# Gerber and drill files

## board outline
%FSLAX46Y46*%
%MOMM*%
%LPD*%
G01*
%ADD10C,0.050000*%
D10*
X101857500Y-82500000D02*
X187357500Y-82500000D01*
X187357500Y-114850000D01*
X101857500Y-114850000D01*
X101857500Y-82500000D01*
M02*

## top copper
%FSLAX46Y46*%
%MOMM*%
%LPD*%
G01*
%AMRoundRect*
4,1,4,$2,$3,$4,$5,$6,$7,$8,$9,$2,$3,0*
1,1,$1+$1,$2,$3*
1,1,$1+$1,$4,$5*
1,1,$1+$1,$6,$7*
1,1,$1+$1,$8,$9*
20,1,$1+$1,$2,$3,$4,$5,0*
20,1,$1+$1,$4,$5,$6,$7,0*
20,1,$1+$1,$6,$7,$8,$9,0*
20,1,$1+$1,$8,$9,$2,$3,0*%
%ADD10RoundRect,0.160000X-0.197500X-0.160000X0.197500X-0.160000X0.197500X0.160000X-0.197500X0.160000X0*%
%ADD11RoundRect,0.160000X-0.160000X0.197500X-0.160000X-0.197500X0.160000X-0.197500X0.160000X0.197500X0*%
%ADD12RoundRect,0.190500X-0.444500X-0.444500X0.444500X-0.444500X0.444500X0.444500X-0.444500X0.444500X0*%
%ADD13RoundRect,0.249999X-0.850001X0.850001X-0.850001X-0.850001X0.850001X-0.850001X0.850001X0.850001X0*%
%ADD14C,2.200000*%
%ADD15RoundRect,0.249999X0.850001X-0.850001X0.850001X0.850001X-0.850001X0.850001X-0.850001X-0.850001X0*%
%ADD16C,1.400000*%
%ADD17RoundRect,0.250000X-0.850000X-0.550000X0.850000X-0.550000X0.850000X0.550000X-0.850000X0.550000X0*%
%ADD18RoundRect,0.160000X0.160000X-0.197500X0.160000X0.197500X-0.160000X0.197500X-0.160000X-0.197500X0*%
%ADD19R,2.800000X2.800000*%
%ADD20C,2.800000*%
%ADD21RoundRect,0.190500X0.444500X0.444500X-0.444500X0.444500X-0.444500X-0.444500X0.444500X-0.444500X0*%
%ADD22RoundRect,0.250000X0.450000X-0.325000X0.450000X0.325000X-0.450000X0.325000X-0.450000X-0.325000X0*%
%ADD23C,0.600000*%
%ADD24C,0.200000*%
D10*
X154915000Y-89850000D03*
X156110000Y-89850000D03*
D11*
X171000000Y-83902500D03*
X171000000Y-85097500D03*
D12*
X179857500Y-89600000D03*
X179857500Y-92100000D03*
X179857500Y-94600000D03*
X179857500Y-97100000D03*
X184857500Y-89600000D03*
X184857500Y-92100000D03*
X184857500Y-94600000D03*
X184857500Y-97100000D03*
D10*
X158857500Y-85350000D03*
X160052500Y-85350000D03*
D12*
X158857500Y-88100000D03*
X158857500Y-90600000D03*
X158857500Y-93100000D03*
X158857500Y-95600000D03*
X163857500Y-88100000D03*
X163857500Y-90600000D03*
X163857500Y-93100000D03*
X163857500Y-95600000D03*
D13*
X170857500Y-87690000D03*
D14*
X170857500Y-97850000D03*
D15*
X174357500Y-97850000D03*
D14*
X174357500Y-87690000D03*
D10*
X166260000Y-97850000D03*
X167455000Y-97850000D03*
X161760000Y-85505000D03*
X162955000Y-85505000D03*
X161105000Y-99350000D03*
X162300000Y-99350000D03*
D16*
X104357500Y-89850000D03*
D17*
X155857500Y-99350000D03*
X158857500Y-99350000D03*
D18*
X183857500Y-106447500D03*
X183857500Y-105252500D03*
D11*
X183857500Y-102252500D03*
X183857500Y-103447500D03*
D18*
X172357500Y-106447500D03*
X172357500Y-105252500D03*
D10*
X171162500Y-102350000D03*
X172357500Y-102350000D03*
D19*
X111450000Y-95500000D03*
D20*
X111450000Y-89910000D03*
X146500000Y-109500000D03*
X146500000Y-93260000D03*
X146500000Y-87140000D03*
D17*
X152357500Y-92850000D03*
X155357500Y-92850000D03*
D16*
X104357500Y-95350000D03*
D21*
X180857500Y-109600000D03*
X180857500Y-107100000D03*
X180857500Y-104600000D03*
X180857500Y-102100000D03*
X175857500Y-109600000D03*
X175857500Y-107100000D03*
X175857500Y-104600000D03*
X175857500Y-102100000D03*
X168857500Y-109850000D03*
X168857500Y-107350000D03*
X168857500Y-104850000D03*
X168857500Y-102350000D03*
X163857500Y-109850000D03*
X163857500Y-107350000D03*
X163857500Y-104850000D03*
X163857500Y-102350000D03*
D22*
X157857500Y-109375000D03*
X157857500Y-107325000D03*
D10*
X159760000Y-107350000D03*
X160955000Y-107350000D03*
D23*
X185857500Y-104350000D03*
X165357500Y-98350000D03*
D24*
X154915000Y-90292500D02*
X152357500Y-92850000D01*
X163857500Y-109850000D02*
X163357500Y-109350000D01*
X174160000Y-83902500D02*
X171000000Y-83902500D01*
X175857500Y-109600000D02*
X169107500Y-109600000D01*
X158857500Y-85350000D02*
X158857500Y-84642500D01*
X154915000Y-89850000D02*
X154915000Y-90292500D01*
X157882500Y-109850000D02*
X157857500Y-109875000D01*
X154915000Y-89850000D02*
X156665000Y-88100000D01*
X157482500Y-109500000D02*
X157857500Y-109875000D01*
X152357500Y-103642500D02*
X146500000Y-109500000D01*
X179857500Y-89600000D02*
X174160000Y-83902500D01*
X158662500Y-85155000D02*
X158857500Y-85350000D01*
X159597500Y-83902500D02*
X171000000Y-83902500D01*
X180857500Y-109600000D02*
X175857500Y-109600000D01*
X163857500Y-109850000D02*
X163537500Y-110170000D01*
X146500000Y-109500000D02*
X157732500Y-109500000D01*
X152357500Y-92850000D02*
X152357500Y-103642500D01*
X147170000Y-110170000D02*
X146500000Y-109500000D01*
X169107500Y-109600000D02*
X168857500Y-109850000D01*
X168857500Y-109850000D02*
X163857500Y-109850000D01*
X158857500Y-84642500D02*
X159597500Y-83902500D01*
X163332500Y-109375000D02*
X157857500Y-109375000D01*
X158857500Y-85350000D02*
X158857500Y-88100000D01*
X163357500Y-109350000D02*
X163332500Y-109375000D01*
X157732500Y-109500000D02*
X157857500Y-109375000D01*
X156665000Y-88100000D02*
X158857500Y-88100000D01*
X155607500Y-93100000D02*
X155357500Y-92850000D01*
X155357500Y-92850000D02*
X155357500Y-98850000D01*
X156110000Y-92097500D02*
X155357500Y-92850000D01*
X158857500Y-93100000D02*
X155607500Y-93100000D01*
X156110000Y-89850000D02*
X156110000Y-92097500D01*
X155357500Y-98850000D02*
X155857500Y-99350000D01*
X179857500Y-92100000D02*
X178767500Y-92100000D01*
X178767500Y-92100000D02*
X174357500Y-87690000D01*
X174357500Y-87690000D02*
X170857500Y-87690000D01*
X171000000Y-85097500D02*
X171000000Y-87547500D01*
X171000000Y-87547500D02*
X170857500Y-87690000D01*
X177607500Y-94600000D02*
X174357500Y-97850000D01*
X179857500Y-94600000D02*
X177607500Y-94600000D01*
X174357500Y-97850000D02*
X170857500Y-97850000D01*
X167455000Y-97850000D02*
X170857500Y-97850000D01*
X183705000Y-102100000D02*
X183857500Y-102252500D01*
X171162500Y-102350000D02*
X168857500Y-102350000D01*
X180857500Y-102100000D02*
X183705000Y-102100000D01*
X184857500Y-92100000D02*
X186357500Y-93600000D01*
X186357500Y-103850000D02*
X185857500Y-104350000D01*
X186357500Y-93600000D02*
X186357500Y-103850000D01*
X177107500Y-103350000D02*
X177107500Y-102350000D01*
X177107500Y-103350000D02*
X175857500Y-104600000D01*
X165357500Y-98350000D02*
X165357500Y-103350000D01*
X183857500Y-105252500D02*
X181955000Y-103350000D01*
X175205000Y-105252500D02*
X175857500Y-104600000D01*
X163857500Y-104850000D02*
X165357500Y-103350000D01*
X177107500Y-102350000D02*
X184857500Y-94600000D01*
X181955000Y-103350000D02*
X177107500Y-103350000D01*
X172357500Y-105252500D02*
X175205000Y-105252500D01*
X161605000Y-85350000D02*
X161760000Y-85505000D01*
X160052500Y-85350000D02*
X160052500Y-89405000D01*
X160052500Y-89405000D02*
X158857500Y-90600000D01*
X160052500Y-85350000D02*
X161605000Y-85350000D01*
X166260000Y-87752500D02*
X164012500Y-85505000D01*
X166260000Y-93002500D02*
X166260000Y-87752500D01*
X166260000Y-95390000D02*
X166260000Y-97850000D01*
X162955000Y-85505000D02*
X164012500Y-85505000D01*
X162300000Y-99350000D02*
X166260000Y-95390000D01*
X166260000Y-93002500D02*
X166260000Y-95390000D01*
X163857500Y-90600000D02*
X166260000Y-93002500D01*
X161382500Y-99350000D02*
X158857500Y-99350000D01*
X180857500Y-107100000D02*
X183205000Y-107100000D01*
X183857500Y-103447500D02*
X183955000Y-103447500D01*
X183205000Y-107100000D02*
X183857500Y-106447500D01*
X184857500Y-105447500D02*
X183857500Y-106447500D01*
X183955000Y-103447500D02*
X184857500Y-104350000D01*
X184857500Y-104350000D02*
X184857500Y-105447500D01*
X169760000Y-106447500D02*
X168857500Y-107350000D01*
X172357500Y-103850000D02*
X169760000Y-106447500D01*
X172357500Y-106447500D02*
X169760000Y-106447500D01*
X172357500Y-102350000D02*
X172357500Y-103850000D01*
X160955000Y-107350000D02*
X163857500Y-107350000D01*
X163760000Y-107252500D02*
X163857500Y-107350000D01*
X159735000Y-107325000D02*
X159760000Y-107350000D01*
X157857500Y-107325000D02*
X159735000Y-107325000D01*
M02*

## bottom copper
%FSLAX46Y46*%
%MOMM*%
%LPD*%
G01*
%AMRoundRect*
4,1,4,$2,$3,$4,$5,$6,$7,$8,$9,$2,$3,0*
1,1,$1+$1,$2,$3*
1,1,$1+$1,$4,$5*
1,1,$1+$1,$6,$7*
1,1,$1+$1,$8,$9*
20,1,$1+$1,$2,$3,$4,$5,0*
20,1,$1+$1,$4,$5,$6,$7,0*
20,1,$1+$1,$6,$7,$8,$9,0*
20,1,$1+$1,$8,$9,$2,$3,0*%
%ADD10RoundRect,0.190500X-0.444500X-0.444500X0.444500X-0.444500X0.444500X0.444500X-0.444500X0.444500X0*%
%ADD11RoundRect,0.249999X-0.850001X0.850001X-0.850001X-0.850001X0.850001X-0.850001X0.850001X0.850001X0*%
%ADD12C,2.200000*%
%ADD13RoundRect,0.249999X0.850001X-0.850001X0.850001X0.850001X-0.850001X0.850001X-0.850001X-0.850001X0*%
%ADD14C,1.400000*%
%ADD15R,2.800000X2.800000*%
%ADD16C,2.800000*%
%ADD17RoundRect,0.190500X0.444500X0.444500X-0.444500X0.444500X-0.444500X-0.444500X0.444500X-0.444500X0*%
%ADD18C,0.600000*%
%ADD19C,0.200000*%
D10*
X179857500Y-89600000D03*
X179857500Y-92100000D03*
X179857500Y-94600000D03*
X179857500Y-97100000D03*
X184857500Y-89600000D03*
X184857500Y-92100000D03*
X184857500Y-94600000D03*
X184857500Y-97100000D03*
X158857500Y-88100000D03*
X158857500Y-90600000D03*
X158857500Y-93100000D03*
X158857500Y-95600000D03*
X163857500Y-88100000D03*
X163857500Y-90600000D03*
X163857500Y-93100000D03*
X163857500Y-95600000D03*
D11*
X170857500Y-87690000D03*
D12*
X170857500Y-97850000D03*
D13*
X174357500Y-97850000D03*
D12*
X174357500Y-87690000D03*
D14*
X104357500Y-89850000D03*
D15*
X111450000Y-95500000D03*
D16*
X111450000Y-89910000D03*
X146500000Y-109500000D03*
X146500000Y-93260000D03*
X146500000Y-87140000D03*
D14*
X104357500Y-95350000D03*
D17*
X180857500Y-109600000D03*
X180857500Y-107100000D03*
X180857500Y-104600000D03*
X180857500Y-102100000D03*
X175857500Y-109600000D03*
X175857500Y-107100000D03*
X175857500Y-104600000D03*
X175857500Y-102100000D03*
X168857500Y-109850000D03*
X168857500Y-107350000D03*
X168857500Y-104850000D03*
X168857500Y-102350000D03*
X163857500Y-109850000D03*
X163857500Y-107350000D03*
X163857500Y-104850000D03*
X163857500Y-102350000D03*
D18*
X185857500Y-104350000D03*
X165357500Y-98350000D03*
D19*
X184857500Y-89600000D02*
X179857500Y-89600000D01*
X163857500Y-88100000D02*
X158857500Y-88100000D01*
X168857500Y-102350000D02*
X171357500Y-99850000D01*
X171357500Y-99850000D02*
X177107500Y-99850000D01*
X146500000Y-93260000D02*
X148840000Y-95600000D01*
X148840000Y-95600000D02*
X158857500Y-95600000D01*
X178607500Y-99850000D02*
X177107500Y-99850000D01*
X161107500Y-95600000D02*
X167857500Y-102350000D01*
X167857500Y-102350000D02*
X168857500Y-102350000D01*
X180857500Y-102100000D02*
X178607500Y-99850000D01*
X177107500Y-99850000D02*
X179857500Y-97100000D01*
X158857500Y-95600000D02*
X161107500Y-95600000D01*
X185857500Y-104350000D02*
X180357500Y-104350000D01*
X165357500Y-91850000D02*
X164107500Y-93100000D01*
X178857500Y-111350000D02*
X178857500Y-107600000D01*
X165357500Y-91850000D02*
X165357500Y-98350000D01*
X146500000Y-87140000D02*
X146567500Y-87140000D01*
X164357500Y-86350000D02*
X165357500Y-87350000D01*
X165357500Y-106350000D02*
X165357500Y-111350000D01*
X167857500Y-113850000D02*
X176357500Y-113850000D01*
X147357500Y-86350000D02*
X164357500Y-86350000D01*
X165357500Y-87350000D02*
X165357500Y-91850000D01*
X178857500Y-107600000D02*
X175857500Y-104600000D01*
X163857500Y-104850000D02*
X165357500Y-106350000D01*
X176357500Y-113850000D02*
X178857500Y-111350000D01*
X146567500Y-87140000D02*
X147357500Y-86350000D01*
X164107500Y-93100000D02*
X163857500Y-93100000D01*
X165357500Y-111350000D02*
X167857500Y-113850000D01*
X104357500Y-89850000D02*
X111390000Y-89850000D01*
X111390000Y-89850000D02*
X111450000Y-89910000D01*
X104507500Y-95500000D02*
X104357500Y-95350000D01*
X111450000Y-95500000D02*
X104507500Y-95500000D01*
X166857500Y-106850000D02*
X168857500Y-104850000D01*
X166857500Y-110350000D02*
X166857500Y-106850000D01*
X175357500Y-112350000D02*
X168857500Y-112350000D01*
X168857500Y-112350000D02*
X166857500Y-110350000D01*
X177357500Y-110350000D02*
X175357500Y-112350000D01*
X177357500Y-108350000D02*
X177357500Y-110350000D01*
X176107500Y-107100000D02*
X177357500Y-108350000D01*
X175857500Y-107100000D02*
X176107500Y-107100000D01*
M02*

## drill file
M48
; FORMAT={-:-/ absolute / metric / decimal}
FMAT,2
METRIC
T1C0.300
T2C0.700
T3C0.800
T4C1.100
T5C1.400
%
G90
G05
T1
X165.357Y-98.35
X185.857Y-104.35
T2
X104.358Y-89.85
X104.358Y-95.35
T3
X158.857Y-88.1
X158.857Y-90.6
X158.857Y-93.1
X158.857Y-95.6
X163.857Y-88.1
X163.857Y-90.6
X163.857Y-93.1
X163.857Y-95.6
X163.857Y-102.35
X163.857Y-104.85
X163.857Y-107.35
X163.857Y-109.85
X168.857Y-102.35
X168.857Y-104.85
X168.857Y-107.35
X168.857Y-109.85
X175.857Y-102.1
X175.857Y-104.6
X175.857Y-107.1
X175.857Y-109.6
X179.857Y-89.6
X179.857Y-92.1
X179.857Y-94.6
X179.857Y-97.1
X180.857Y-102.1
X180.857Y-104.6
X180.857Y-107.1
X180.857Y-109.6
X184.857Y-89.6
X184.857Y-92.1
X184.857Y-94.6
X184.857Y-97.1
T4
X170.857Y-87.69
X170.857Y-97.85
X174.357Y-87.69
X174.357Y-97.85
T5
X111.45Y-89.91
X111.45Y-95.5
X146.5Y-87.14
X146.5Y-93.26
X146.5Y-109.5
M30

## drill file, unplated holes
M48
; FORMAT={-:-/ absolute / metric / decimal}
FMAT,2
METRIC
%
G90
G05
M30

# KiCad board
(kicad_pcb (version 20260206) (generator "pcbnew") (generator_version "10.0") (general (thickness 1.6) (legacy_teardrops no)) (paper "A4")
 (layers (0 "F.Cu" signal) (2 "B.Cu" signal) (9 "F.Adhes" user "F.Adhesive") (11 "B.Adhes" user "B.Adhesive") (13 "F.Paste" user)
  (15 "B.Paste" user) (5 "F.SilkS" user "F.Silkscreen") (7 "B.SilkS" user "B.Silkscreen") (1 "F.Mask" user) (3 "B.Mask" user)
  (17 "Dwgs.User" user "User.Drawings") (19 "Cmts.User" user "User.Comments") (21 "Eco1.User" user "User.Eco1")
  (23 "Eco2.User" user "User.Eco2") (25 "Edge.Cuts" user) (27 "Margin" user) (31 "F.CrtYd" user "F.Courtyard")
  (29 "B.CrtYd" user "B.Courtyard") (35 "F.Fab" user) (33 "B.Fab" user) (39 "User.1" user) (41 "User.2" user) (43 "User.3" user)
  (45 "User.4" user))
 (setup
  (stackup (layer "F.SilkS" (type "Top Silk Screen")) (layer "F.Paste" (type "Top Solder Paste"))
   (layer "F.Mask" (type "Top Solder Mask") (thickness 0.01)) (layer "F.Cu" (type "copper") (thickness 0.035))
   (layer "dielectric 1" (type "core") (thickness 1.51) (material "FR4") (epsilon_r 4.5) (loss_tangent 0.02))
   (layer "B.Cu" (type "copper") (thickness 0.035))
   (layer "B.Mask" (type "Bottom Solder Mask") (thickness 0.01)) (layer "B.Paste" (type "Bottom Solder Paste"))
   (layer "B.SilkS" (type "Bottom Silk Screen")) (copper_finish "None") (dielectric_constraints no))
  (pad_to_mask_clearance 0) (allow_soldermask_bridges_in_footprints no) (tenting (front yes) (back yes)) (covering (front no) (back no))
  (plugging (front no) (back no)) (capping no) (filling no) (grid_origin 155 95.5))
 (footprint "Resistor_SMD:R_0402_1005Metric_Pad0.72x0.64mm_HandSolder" (layer "F.Cu") (at 155.5125 89.85)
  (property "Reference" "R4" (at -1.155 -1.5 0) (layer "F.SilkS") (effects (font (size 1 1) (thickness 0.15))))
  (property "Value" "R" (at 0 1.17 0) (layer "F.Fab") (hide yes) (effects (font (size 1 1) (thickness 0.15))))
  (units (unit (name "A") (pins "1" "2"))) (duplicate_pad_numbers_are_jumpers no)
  (pad "1" smd roundrect (at -0.5975 0) (size 0.715 0.64) (layers "F.Cu" "F.Mask" "F.Paste") (roundrect_rratio 0.25) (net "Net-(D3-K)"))
  (pad "2" smd roundrect (at 0.5975 0) (size 0.715 0.64) (layers "F.Cu" "F.Mask" "F.Paste") (roundrect_rratio 0.25) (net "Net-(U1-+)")))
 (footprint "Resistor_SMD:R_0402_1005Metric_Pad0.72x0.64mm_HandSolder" (layer "F.Cu") (at 171 84.5 -90)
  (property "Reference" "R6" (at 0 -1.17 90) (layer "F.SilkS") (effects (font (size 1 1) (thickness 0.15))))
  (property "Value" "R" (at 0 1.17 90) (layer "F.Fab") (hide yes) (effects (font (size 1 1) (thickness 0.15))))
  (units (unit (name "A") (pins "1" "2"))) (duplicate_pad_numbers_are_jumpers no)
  (pad "1" smd roundrect (at -0.5975 0 270) (size 0.715 0.64) (layers "F.Cu" "F.Mask" "F.Paste") (roundrect_rratio 0.25) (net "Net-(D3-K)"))
  (pad "2" smd roundrect (at 0.5975 0 270) (size 0.715 0.64) (layers "F.Cu" "F.Mask" "F.Paste") (roundrect_rratio 0.25) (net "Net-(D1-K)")))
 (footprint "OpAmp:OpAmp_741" (layer "F.Cu") (at 182.3575 96.1)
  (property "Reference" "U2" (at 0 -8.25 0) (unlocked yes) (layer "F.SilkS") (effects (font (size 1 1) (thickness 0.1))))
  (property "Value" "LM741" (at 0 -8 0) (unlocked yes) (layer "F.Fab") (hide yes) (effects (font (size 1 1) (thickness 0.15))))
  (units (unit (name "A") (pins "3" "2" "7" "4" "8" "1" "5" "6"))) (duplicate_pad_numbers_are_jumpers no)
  (pad "1" thru_hole roundrect (at -2.5 -6.5) (size 1.27 1.27) (drill 0.8) (layers "*.Cu" "*.Mask") (remove_unused_layers no)
   (roundrect_rratio 0.15) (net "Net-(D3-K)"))
  (pad "2" thru_hole roundrect (at -2.5 -4) (size 1.27 1.27) (drill 0.8) (layers "*.Cu" "*.Mask") (remove_unused_layers no)
   (roundrect_rratio 0.15) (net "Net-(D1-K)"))
  (pad "3" thru_hole roundrect (at -2.5 -1.5) (size 1.27 1.27) (drill 0.8) (layers "*.Cu" "*.Mask") (remove_unused_layers no)
   (roundrect_rratio 0.15) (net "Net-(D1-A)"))
  (pad "4" thru_hole roundrect (at -2.5 1) (size 1.27 1.27) (drill 0.8) (layers "*.Cu" "*.Mask") (remove_unused_layers no)
   (roundrect_rratio 0.15) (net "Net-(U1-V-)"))
  (pad "5" thru_hole roundrect (at 2.5 -6.5) (size 1.27 1.27) (drill 0.8) (layers "*.Cu" "*.Mask") (remove_unused_layers no)
   (roundrect_rratio 0.15) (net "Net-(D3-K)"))
  (pad "6" thru_hole roundrect (at 2.5 -4) (size 1.27 1.27) (drill 0.8) (layers "*.Cu" "*.Mask") (remove_unused_layers no)
   (roundrect_rratio 0.15) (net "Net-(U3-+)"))
  (pad "7" thru_hole roundrect (at 2.5 -1.5) (size 1.27 1.27) (drill 0.8) (layers "*.Cu" "*.Mask") (remove_unused_layers no)
   (roundrect_rratio 0.15) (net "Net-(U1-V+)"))
  (pad "8" thru_hole roundrect (at 2.5 1) (size 1.27 1.27) (drill 0.8) (layers "*.Cu" "*.Mask") (remove_unused_layers no)
   (roundrect_rratio 0.15) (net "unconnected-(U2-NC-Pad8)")))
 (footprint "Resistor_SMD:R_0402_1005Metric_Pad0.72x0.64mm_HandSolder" (layer "F.Cu") (at 159.455 85.35)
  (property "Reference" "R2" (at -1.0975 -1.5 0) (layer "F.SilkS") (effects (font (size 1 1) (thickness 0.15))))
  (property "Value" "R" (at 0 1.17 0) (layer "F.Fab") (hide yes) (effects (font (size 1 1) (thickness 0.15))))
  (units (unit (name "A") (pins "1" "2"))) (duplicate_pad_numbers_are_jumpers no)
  (pad "1" smd roundrect (at -0.5975 0) (size 0.715 0.64) (layers "F.Cu" "F.Mask" "F.Paste") (roundrect_rratio 0.25) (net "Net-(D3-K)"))
  (pad "2" smd roundrect (at 0.5975 0) (size 0.715 0.64) (layers "F.Cu" "F.Mask" "F.Paste") (roundrect_rratio 0.25) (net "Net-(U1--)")))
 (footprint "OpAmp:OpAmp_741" (layer "F.Cu") (at 161.3575 94.6)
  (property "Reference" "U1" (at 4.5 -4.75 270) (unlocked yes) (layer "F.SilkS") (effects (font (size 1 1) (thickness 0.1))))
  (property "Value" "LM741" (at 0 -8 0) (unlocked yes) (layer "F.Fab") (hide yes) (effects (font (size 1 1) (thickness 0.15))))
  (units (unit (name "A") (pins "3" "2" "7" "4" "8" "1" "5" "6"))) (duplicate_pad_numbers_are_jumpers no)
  (pad "1" thru_hole roundrect (at -2.5 -6.5) (size 1.27 1.27) (drill 0.8) (layers "*.Cu" "*.Mask") (remove_unused_layers no)
   (roundrect_rratio 0.15) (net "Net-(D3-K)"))
  (pad "2" thru_hole roundrect (at -2.5 -4) (size 1.27 1.27) (drill 0.8) (layers "*.Cu" "*.Mask") (remove_unused_layers no)
   (roundrect_rratio 0.15) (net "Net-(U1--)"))
  (pad "3" thru_hole roundrect (at -2.5 -1.5) (size 1.27 1.27) (drill 0.8) (layers "*.Cu" "*.Mask") (remove_unused_layers no)
   (roundrect_rratio 0.15) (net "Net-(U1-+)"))
  (pad "4" thru_hole roundrect (at -2.5 1) (size 1.27 1.27) (drill 0.8) (layers "*.Cu" "*.Mask") (remove_unused_layers no)
   (roundrect_rratio 0.15) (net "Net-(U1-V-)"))
  (pad "5" thru_hole roundrect (at 2.5 -6.5) (size 1.27 1.27) (drill 0.8) (layers "*.Cu" "*.Mask") (remove_unused_layers no)
   (roundrect_rratio 0.15) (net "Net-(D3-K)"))
  (pad "6" thru_hole roundrect (at 2.5 -4) (size 1.27 1.27) (drill 0.8) (layers "*.Cu" "*.Mask") (remove_unused_layers no)
   (roundrect_rratio 0.15) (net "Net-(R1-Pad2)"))
  (pad "7" thru_hole roundrect (at 2.5 -1.5) (size 1.27 1.27) (drill 0.8) (layers "*.Cu" "*.Mask") (remove_unused_layers no)
   (roundrect_rratio 0.15) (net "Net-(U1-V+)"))
  (pad "8" thru_hole roundrect (at 2.5 1) (size 1.27 1.27) (drill 0.8) (layers "*.Cu" "*.Mask") (remove_unused_layers no)
   (roundrect_rratio 0.15) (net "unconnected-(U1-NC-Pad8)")))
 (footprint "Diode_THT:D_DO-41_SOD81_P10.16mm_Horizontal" (layer "F.Cu") (at 170.8575 87.69 -90)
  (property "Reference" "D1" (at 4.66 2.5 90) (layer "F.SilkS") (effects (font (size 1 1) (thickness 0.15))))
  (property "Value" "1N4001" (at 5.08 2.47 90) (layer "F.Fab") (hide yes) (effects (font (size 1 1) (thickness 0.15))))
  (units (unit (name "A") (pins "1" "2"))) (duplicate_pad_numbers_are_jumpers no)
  (pad "1" thru_hole roundrect (at 0 0 270) (size 2.2 2.2) (drill 1.1) (layers "*.Cu" "*.Mask") (remove_unused_layers no)
   (roundrect_rratio 0.113636) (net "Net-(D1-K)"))
  (pad "2" thru_hole circle (at 10.16 0 270) (size 2.2 2.2) (drill 1.1) (layers "*.Cu" "*.Mask") (remove_unused_layers no)
   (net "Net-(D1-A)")))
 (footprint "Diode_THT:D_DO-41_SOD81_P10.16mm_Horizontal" (layer "F.Cu") (at 174.3575 97.85 90)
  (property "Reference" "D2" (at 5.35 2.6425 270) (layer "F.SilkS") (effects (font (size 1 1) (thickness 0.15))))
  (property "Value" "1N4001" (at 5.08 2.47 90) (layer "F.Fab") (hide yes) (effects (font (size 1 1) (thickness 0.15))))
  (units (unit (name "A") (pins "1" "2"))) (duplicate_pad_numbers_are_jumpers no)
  (pad "1" thru_hole roundrect (at 0 0 90) (size 2.2 2.2) (drill 1.1) (layers "*.Cu" "*.Mask") (remove_unused_layers no)
   (roundrect_rratio 0.113636) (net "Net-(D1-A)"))
  (pad "2" thru_hole circle (at 10.16 0 90) (size 2.2 2.2) (drill 1.1) (layers "*.Cu" "*.Mask") (remove_unused_layers no) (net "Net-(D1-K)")))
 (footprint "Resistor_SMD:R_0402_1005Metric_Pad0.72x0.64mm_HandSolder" (layer "F.Cu") (at 166.8575 97.85)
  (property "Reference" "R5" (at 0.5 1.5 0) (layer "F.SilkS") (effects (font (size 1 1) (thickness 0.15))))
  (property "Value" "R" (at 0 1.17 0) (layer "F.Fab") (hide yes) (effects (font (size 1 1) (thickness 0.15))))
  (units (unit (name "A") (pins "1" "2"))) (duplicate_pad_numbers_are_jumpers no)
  (pad "1" smd roundrect (at -0.5975 0) (size 0.715 0.64) (layers "F.Cu" "F.Mask" "F.Paste") (roundrect_rratio 0.25) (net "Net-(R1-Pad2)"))
  (pad "2" smd roundrect (at 0.5975 0) (size 0.715 0.64) (layers "F.Cu" "F.Mask" "F.Paste") (roundrect_rratio 0.25) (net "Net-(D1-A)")))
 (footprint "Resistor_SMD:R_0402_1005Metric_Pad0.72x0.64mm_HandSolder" (layer "F.Cu") (at 162.3575 85.505)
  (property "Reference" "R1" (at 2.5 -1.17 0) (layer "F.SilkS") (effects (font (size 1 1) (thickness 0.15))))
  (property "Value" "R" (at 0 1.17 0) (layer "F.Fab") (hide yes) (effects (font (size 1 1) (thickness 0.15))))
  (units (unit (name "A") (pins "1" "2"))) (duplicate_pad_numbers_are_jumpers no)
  (pad "1" smd roundrect (at -0.5975 0) (size 0.715 0.64) (layers "F.Cu" "F.Mask" "F.Paste") (roundrect_rratio 0.25) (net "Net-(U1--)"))
  (pad "2" smd roundrect (at 0.5975 0) (size 0.715 0.64) (layers "F.Cu" "F.Mask" "F.Paste") (roundrect_rratio 0.25) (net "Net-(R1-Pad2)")))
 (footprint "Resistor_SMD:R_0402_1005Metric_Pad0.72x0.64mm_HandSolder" (layer "F.Cu") (at 161.7025 99.35)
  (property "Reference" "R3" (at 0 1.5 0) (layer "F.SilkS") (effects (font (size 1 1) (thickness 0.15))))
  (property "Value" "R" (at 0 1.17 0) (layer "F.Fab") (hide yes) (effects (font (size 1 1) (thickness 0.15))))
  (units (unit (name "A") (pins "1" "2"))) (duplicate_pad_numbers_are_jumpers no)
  (pad "1" smd roundrect (at -0.5975 0) (size 0.715 0.64) (layers "F.Cu" "F.Mask" "F.Paste") (roundrect_rratio 0.25) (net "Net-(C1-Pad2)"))
  (pad "2" smd roundrect (at 0.5975 0) (size 0.715 0.64) (layers "F.Cu" "F.Mask" "F.Paste") (roundrect_rratio 0.25) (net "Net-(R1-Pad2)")))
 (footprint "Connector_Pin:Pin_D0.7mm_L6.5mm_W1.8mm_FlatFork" (layer "F.Cu") (at 104.3575 89.85)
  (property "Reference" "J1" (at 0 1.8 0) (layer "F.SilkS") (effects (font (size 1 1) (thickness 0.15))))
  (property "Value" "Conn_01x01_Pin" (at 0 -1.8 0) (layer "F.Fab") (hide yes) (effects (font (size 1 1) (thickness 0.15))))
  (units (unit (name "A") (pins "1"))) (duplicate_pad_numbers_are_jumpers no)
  (pad "1" thru_hole circle (at 0 0) (size 1.4 1.4) (drill 0.7) (layers "*.Cu" "*.Mask") (remove_unused_layers no) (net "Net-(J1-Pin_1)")))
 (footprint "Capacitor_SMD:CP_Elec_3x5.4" (layer "F.Cu") (at 157.3575 99.35)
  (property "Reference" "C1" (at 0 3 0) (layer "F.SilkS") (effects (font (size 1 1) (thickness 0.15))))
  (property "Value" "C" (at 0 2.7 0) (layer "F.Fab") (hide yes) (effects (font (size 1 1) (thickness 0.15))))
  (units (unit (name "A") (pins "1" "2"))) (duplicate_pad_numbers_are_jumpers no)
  (pad "1" smd roundrect (at -1.5 0) (size 2.2 1.6) (layers "F.Cu" "F.Mask" "F.Paste") (roundrect_rratio 0.15625) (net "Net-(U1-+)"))
  (pad "2" smd roundrect (at 1.5 0) (size 2.2 1.6) (layers "F.Cu" "F.Mask" "F.Paste") (roundrect_rratio 0.15625) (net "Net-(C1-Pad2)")))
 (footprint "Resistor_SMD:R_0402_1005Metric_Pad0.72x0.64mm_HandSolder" (layer "F.Cu") (at 183.8575 105.85 90)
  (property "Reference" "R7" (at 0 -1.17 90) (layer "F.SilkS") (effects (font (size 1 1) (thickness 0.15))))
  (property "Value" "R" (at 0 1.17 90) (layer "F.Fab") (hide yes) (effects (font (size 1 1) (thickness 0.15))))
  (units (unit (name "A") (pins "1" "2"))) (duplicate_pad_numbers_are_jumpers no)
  (pad "1" smd roundrect (at -0.5975 0 90) (size 0.715 0.64) (layers "F.Cu" "F.Mask" "F.Paste") (roundrect_rratio 0.25) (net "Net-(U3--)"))
  (pad "2" smd roundrect (at 0.5975 0 90) (size 0.715 0.64) (layers "F.Cu" "F.Mask" "F.Paste") (roundrect_rratio 0.25) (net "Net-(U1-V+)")))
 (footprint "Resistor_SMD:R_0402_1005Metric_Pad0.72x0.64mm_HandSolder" (layer "F.Cu") (at 183.8575 102.85 -90)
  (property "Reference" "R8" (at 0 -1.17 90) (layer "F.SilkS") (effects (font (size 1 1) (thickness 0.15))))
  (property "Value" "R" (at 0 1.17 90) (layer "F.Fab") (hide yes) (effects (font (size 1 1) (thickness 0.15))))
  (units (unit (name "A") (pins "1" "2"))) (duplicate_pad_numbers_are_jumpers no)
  (pad "1" smd roundrect (at -0.5975 0 270) (size 0.715 0.64) (layers "F.Cu" "F.Mask" "F.Paste") (roundrect_rratio 0.25) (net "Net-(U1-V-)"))
  (pad "2" smd roundrect (at 0.5975 0 270) (size 0.715 0.64) (layers "F.Cu" "F.Mask" "F.Paste") (roundrect_rratio 0.25) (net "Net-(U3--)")))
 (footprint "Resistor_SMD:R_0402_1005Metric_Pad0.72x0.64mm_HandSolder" (layer "F.Cu") (at 172.3575 105.85 90)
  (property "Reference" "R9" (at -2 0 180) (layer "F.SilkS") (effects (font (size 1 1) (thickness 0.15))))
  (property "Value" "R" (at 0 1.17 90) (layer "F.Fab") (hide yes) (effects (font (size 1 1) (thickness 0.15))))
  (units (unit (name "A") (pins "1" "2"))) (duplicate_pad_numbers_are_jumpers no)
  (pad "1" smd roundrect (at -0.5975 0 90) (size 0.715 0.64) (layers "F.Cu" "F.Mask" "F.Paste") (roundrect_rratio 0.25) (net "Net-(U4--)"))
  (pad "2" smd roundrect (at 0.5975 0 90) (size 0.715 0.64) (layers "F.Cu" "F.Mask" "F.Paste") (roundrect_rratio 0.25) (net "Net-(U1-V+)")))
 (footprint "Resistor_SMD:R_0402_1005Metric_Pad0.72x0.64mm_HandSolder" (layer "F.Cu") (at 171.76 102.35)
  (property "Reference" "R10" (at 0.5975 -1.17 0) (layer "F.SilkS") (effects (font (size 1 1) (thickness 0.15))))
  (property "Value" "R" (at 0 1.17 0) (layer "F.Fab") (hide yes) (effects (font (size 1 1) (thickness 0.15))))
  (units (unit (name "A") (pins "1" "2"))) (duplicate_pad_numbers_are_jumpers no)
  (pad "1" smd roundrect (at -0.5975 0) (size 0.715 0.64) (layers "F.Cu" "F.Mask" "F.Paste") (roundrect_rratio 0.25) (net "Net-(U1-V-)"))
  (pad "2" smd roundrect (at 0.5975 0) (size 0.715 0.64) (layers "F.Cu" "F.Mask" "F.Paste") (roundrect_rratio 0.25) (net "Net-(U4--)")))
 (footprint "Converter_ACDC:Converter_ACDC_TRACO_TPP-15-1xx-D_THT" (layer "F.Cu") (at 111.45 95.5)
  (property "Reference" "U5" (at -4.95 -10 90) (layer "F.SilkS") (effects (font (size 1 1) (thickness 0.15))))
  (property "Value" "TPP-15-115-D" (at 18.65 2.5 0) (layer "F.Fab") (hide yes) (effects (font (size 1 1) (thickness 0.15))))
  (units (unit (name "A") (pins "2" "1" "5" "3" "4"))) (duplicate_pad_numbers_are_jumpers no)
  (pad "1" thru_hole rect (at 0 0) (size 2.8 2.8) (drill 1.4) (layers "*.Cu" "*.Mask") (remove_unused_layers no) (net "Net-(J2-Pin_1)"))
  (pad "2" thru_hole circle (at 0 -5.59) (size 2.8 2.8) (drill 1.4) (layers "*.Cu" "*.Mask") (remove_unused_layers no)
   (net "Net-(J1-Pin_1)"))
  (pad "3" thru_hole circle (at 35.05 14) (size 2.8 2.8) (drill 1.4) (layers "*.Cu" "*.Mask") (remove_unused_layers no) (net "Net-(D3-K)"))
  (pad "4" thru_hole circle (at 35.05 -2.24) (size 2.8 2.8) (drill 1.4) (layers "*.Cu" "*.Mask") (remove_unused_layers no)
   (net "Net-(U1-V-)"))
  (pad "5" thru_hole circle (at 35.05 -8.36) (size 2.8 2.8) (drill 1.4) (layers "*.Cu" "*.Mask") (remove_unused_layers no)
   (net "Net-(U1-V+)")))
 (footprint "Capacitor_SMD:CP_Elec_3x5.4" (layer "F.Cu") (at 153.8575 92.85)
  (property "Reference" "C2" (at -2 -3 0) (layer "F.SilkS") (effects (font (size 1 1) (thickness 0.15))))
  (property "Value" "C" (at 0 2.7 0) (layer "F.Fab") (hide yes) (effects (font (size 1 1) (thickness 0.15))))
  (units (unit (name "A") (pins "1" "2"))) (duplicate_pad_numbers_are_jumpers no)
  (pad "1" smd roundrect (at -1.5 0) (size 2.2 1.6) (layers "F.Cu" "F.Mask" "F.Paste") (roundrect_rratio 0.15625) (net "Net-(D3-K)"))
  (pad "2" smd roundrect (at 1.5 0) (size 2.2 1.6) (layers "F.Cu" "F.Mask" "F.Paste") (roundrect_rratio 0.15625) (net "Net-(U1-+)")))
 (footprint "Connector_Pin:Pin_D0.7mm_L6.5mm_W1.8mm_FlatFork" (layer "F.Cu") (at 104.3575 95.35)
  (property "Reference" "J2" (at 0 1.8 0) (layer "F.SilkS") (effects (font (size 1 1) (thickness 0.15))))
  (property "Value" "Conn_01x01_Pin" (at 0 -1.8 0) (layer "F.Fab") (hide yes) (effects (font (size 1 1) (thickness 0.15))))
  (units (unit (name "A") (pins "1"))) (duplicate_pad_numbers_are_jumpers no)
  (pad "1" thru_hole circle (at 0 0) (size 1.4 1.4) (drill 0.7) (layers "*.Cu" "*.Mask") (remove_unused_layers no) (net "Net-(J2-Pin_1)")))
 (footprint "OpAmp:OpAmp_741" (layer "F.Cu") (at 178.3575 103.1 180)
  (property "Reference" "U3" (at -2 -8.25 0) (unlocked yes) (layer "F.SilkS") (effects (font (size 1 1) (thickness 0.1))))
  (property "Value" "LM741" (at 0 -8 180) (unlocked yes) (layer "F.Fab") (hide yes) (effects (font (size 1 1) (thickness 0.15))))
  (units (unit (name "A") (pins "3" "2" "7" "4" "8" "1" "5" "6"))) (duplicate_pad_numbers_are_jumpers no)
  (pad "1" thru_hole roundrect (at -2.5 -6.5 180) (size 1.27 1.27) (drill 0.8) (layers "*.Cu" "*.Mask") (remove_unused_layers no)
   (roundrect_rratio 0.15) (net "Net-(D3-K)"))
  (pad "2" thru_hole roundrect (at -2.5 -4 180) (size 1.27 1.27) (drill 0.8) (layers "*.Cu" "*.Mask") (remove_unused_layers no)
   (roundrect_rratio 0.15) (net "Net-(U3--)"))
  (pad "3" thru_hole roundrect (at -2.5 -1.5 180) (size 1.27 1.27) (drill 0.8) (layers "*.Cu" "*.Mask") (remove_unused_layers no)
   (roundrect_rratio 0.15) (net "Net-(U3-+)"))
  (pad "4" thru_hole roundrect (at -2.5 1 180) (size 1.27 1.27) (drill 0.8) (layers "*.Cu" "*.Mask") (remove_unused_layers no)
   (roundrect_rratio 0.15) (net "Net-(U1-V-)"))
  (pad "5" thru_hole roundrect (at 2.5 -6.5 180) (size 1.27 1.27) (drill 0.8) (layers "*.Cu" "*.Mask") (remove_unused_layers no)
   (roundrect_rratio 0.15) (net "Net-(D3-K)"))
  (pad "6" thru_hole roundrect (at 2.5 -4 180) (size 1.27 1.27) (drill 0.8) (layers "*.Cu" "*.Mask") (remove_unused_layers no)
   (roundrect_rratio 0.15) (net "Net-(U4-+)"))
  (pad "7" thru_hole roundrect (at 2.5 -1.5 180) (size 1.27 1.27) (drill 0.8) (layers "*.Cu" "*.Mask") (remove_unused_layers no)
   (roundrect_rratio 0.15) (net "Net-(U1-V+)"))
  (pad "8" thru_hole roundrect (at 2.5 1 180) (size 1.27 1.27) (drill 0.8) (layers "*.Cu" "*.Mask") (remove_unused_layers no)
   (roundrect_rratio 0.15) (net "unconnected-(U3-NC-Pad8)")))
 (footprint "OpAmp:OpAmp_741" (layer "F.Cu") (at 166.3575 103.35 180)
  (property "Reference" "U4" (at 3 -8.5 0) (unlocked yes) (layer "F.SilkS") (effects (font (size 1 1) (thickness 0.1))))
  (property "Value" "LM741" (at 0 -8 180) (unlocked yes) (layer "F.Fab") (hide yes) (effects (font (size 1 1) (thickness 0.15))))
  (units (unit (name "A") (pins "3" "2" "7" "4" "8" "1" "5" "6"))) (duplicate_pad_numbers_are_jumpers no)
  (pad "1" thru_hole roundrect (at -2.5 -6.5 180) (size 1.27 1.27) (drill 0.8) (layers "*.Cu" "*.Mask") (remove_unused_layers no)
   (roundrect_rratio 0.15) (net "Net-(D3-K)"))
  (pad "2" thru_hole roundrect (at -2.5 -4 180) (size 1.27 1.27) (drill 0.8) (layers "*.Cu" "*.Mask") (remove_unused_layers no)
   (roundrect_rratio 0.15) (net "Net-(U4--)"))
  (pad "3" thru_hole roundrect (at -2.5 -1.5 180) (size 1.27 1.27) (drill 0.8) (layers "*.Cu" "*.Mask") (remove_unused_layers no)
   (roundrect_rratio 0.15) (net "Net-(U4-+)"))
  (pad "4" thru_hole roundrect (at -2.5 1 180) (size 1.27 1.27) (drill 0.8) (layers "*.Cu" "*.Mask") (remove_unused_layers no)
   (roundrect_rratio 0.15) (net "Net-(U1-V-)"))
  (pad "5" thru_hole roundrect (at 2.5 -6.5 180) (size 1.27 1.27) (drill 0.8) (layers "*.Cu" "*.Mask") (remove_unused_layers no)
   (roundrect_rratio 0.15) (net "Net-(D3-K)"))
  (pad "6" thru_hole roundrect (at 2.5 -4 180) (size 1.27 1.27) (drill 0.8) (layers "*.Cu" "*.Mask") (remove_unused_layers no)
   (roundrect_rratio 0.15) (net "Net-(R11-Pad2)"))
  (pad "7" thru_hole roundrect (at 2.5 -1.5 180) (size 1.27 1.27) (drill 0.8) (layers "*.Cu" "*.Mask") (remove_unused_layers no)
   (roundrect_rratio 0.15) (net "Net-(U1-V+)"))
  (pad "8" thru_hole roundrect (at 2.5 1 180) (size 1.27 1.27) (drill 0.8) (layers "*.Cu" "*.Mask") (remove_unused_layers no)
   (roundrect_rratio 0.15) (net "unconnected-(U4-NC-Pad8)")))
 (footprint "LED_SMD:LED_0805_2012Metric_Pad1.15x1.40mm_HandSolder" (layer "F.Cu") (at 157.8575 108.35 90)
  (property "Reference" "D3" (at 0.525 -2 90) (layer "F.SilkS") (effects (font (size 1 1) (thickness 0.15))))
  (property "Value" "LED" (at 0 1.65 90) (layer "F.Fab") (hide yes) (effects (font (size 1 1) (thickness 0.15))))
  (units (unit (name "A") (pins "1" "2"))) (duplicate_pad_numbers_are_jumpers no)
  (pad "1" smd roundrect (at -1.025 0 90) (size 1.15 1.4) (layers "F.Cu" "F.Mask" "F.Paste") (roundrect_rratio 0.217391) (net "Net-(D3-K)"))
  (pad "2" smd roundrect (at 1.025 0 90) (size 1.15 1.4) (layers "F.Cu" "F.Mask" "F.Paste") (roundrect_rratio 0.217391) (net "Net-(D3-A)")))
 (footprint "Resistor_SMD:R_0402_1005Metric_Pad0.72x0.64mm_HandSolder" (layer "F.Cu") (at 160.3575 107.35)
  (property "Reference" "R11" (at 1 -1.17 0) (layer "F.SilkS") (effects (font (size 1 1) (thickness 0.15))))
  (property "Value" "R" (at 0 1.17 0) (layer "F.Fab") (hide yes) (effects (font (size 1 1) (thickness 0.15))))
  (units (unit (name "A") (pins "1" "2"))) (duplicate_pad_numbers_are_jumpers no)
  (pad "1" smd roundrect (at -0.5975 0) (size 0.715 0.64) (layers "F.Cu" "F.Mask" "F.Paste") (roundrect_rratio 0.25) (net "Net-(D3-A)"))
  (pad "2" smd roundrect (at 0.5975 0) (size 0.715 0.64) (layers "F.Cu" "F.Mask" "F.Paste") (roundrect_rratio 0.25) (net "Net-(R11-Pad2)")))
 (gr_rect (start 101.8575 82.5) (end 187.3575 114.85) (stroke (width 0.05) (type default)) (fill no) (layer "Edge.Cuts"))
 (segment (start 154.915 90.2925) (end 152.3575 92.85) (width 0.2) (layer "F.Cu") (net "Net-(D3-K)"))
 (segment (start 163.8575 109.85) (end 163.3575 109.35) (width 0.2) (layer "F.Cu") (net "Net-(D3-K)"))
 (segment (start 174.16 83.9025) (end 171 83.9025) (width 0.2) (layer "F.Cu") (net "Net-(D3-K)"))
 (segment (start 175.8575 109.6) (end 169.1075 109.6) (width 0.2) (layer "F.Cu") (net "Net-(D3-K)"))
 (segment (start 158.8575 85.35) (end 158.8575 84.6425) (width 0.2) (layer "F.Cu") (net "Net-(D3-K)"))
 (segment (start 154.915 89.85) (end 154.915 90.2925) (width 0.2) (layer "F.Cu") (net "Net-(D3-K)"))
 (segment (start 157.8825 109.85) (end 157.8575 109.875) (width 0.2) (layer "F.Cu") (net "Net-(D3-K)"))
 (segment (start 154.915 89.85) (end 156.665 88.1) (width 0.2) (layer "F.Cu") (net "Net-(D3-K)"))
 (segment (start 157.4825 109.5) (end 157.8575 109.875) (width 0.2) (layer "F.Cu") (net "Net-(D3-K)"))
 (segment (start 152.3575 103.6425) (end 146.5 109.5) (width 0.2) (layer "F.Cu") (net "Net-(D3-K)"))
 (segment (start 179.8575 89.6) (end 174.16 83.9025) (width 0.2) (layer "F.Cu") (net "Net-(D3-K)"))
 (segment (start 158.6625 85.155) (end 158.8575 85.35) (width 0.2) (layer "F.Cu") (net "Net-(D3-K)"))
 (segment (start 159.5975 83.9025) (end 171 83.9025) (width 0.2) (layer "F.Cu") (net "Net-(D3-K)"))
 (segment (start 180.8575 109.6) (end 175.8575 109.6) (width 0.2) (layer "F.Cu") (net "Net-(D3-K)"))
 (segment (start 163.8575 109.85) (end 163.5375 110.17) (width 0.2) (layer "F.Cu") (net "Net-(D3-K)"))
 (segment (start 146.5 109.5) (end 157.7325 109.5) (width 0.2) (layer "F.Cu") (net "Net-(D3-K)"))
 (segment (start 152.3575 92.85) (end 152.3575 103.6425) (width 0.2) (layer "F.Cu") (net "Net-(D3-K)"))
 (segment (start 147.17 110.17) (end 146.5 109.5) (width 0.2) (layer "F.Cu") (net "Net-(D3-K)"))
 (segment (start 169.1075 109.6) (end 168.8575 109.85) (width 0.2) (layer "F.Cu") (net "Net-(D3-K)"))
 (segment (start 168.8575 109.85) (end 163.8575 109.85) (width 0.2) (layer "F.Cu") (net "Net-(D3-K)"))
 (segment (start 158.8575 84.6425) (end 159.5975 83.9025) (width 0.2) (layer "F.Cu") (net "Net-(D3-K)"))
 (segment (start 163.3325 109.375) (end 157.8575 109.375) (width 0.2) (layer "F.Cu") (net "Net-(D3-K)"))
 (segment (start 158.8575 85.35) (end 158.8575 88.1) (width 0.2) (layer "F.Cu") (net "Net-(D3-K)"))
 (segment (start 163.3575 109.35) (end 163.3325 109.375) (width 0.2) (layer "F.Cu") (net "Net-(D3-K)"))
 (segment (start 157.7325 109.5) (end 157.8575 109.375) (width 0.2) (layer "F.Cu") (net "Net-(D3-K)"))
 (segment (start 156.665 88.1) (end 158.8575 88.1) (width 0.2) (layer "F.Cu") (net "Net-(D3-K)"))
 (segment (start 184.8575 89.6) (end 179.8575 89.6) (width 0.2) (layer "B.Cu") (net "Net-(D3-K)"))
 (segment (start 163.8575 88.1) (end 158.8575 88.1) (width 0.2) (layer "B.Cu") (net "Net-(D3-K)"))
 (segment (start 155.6075 93.1) (end 155.3575 92.85) (width 0.2) (layer "F.Cu") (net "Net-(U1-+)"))
 (segment (start 155.3575 92.85) (end 155.3575 98.85) (width 0.2) (layer "F.Cu") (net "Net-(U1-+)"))
 (segment (start 156.11 92.0975) (end 155.3575 92.85) (width 0.2) (layer "F.Cu") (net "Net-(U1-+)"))
 (segment (start 158.8575 93.1) (end 155.6075 93.1) (width 0.2) (layer "F.Cu") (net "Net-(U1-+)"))
 (segment (start 156.11 89.85) (end 156.11 92.0975) (width 0.2) (layer "F.Cu") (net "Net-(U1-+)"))
 (segment (start 155.3575 98.85) (end 155.8575 99.35) (width 0.2) (layer "F.Cu") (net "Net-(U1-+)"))
 (segment (start 179.8575 92.1) (end 178.7675 92.1) (width 0.2) (layer "F.Cu") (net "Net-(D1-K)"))
 (segment (start 178.7675 92.1) (end 174.3575 87.69) (width 0.2) (layer "F.Cu") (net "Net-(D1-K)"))
 (segment (start 174.3575 87.69) (end 170.8575 87.69) (width 0.2) (layer "F.Cu") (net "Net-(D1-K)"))
 (segment (start 171 85.0975) (end 171 87.5475) (width 0.2) (layer "F.Cu") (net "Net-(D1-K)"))
 (segment (start 171 87.5475) (end 170.8575 87.69) (width 0.2) (layer "F.Cu") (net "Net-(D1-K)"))
 (segment (start 177.6075 94.6) (end 174.3575 97.85) (width 0.2) (layer "F.Cu") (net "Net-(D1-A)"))
 (segment (start 179.8575 94.6) (end 177.6075 94.6) (width 0.2) (layer "F.Cu") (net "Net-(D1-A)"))
 (segment (start 174.3575 97.85) (end 170.8575 97.85) (width 0.2) (layer "F.Cu") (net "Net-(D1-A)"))
 (segment (start 167.455 97.85) (end 170.8575 97.85) (width 0.2) (layer "F.Cu") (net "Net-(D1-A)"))
 (segment (start 183.705 102.1) (end 183.8575 102.2525) (width 0.2) (layer "F.Cu") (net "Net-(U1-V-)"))
 (segment (start 171.1625 102.35) (end 168.8575 102.35) (width 0.2) (layer "F.Cu") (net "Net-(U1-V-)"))
 (segment (start 180.8575 102.1) (end 183.705 102.1) (width 0.2) (layer "F.Cu") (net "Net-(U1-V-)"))
 (segment (start 168.8575 102.35) (end 171.3575 99.85) (width 0.2) (layer "B.Cu") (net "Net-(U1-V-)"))
 (segment (start 171.3575 99.85) (end 177.1075 99.85) (width 0.2) (layer "B.Cu") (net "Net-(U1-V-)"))
 (segment (start 146.5 93.26) (end 148.84 95.6) (width 0.2) (layer "B.Cu") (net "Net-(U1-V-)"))
 (segment (start 148.84 95.6) (end 158.8575 95.6) (width 0.2) (layer "B.Cu") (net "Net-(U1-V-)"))
 (segment (start 178.6075 99.85) (end 177.1075 99.85) (width 0.2) (layer "B.Cu") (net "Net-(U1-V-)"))
 (segment (start 161.1075 95.6) (end 167.8575 102.35) (width 0.2) (layer "B.Cu") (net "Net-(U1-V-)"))
 (segment (start 167.8575 102.35) (end 168.8575 102.35) (width 0.2) (layer "B.Cu") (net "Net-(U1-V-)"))
 (segment (start 180.8575 102.1) (end 178.6075 99.85) (width 0.2) (layer "B.Cu") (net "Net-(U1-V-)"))
 (segment (start 177.1075 99.85) (end 179.8575 97.1) (width 0.2) (layer "B.Cu") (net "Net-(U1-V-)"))
 (segment (start 158.8575 95.6) (end 161.1075 95.6) (width 0.2) (layer "B.Cu") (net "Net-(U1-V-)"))
 (segment (start 184.8575 92.1) (end 186.3575 93.6) (width 0.2) (layer "F.Cu") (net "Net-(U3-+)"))
 (segment (start 186.3575 103.85) (end 185.8575 104.35) (width 0.2) (layer "F.Cu") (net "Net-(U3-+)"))
 (segment (start 186.3575 93.6) (end 186.3575 103.85) (width 0.2) (layer "F.Cu") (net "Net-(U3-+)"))
 (via (at 185.8575 104.35) (size 0.6) (drill 0.3) (layers "F.Cu" "B.Cu") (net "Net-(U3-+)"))
 (segment (start 185.8575 104.35) (end 180.3575 104.35) (width 0.2) (layer "B.Cu") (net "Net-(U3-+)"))
 (segment (start 177.1075 103.35) (end 177.1075 102.35) (width 0.2) (layer "F.Cu") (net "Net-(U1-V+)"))
 (segment (start 177.1075 103.35) (end 175.8575 104.6) (width 0.2) (layer "F.Cu") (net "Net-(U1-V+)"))
 (segment (start 165.3575 98.35) (end 165.3575 103.35) (width 0.2) (layer "F.Cu") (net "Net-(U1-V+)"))
 (segment (start 183.8575 105.2525) (end 181.955 103.35) (width 0.2) (layer "F.Cu") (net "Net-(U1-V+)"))
 (segment (start 175.205 105.2525) (end 175.8575 104.6) (width 0.2) (layer "F.Cu") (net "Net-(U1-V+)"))
 (segment (start 163.8575 104.85) (end 165.3575 103.35) (width 0.2) (layer "F.Cu") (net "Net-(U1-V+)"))
 (segment (start 177.1075 102.35) (end 184.8575 94.6) (width 0.2) (layer "F.Cu") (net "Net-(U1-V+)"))
 (segment (start 181.955 103.35) (end 177.1075 103.35) (width 0.2) (layer "F.Cu") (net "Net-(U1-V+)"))
 (segment (start 172.3575 105.2525) (end 175.205 105.2525) (width 0.2) (layer "F.Cu") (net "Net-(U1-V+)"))
 (via (at 165.3575 98.35) (size 0.6) (drill 0.3) (layers "F.Cu" "B.Cu") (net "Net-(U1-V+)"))
 (segment (start 165.3575 91.85) (end 164.1075 93.1) (width 0.2) (layer "B.Cu") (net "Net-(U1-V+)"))
 (segment (start 178.8575 111.35) (end 178.8575 107.6) (width 0.2) (layer "B.Cu") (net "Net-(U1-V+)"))
 (segment (start 165.3575 91.85) (end 165.3575 98.35) (width 0.2) (layer "B.Cu") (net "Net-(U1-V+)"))
 (segment (start 146.5 87.14) (end 146.5675 87.14) (width 0.2) (layer "B.Cu") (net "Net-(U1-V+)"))
 (segment (start 164.3575 86.35) (end 165.3575 87.35) (width 0.2) (layer "B.Cu") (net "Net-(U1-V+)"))
 (segment (start 165.3575 106.35) (end 165.3575 111.35) (width 0.2) (layer "B.Cu") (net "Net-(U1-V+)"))
 (segment (start 167.8575 113.85) (end 176.3575 113.85) (width 0.2) (layer "B.Cu") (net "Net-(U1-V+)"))
 (segment (start 147.3575 86.35) (end 164.3575 86.35) (width 0.2) (layer "B.Cu") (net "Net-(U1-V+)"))
 (segment (start 165.3575 87.35) (end 165.3575 91.85) (width 0.2) (layer "B.Cu") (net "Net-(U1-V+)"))
 (segment (start 178.8575 107.6) (end 175.8575 104.6) (width 0.2) (layer "B.Cu") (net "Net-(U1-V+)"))
 (segment (start 163.8575 104.85) (end 165.3575 106.35) (width 0.2) (layer "B.Cu") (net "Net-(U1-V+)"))
 (segment (start 176.3575 113.85) (end 178.8575 111.35) (width 0.2) (layer "B.Cu") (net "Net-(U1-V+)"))
 (segment (start 146.5675 87.14) (end 147.3575 86.35) (width 0.2) (layer "B.Cu") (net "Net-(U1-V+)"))
 (segment (start 164.1075 93.1) (end 163.8575 93.1) (width 0.2) (layer "B.Cu") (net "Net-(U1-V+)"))
 (segment (start 165.3575 111.35) (end 167.8575 113.85) (width 0.2) (layer "B.Cu") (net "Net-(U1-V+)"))
 (segment (start 161.605 85.35) (end 161.76 85.505) (width 0.2) (layer "F.Cu") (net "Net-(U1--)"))
 (segment (start 160.0525 85.35) (end 160.0525 89.405) (width 0.2) (layer "F.Cu") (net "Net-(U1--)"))
 (segment (start 160.0525 89.405) (end 158.8575 90.6) (width 0.2) (layer "F.Cu") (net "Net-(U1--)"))
 (segment (start 160.0525 85.35) (end 161.605 85.35) (width 0.2) (layer "F.Cu") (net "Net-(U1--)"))
 (segment (start 166.26 87.7525) (end 164.0125 85.505) (width 0.2) (layer "F.Cu") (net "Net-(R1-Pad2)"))
 (segment (start 166.26 93.0025) (end 166.26 87.7525) (width 0.2) (layer "F.Cu") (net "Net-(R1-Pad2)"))
 (segment (start 166.26 95.39) (end 166.26 97.85) (width 0.2) (layer "F.Cu") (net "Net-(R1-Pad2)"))
 (segment (start 162.955 85.505) (end 164.0125 85.505) (width 0.2) (layer "F.Cu") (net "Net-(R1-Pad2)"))
 (segment (start 162.3 99.35) (end 166.26 95.39) (width 0.2) (layer "F.Cu") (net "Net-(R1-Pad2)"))
 (segment (start 166.26 93.0025) (end 166.26 95.39) (width 0.2) (layer "F.Cu") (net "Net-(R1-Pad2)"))
 (segment (start 163.8575 90.6) (end 166.26 93.0025) (width 0.2) (layer "F.Cu") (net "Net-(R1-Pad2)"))
 (segment (start 161.3825 99.35) (end 158.8575 99.35) (width 0.2) (layer "F.Cu") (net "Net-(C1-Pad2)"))
 (segment (start 104.3575 89.85) (end 111.39 89.85) (width 0.2) (layer "B.Cu") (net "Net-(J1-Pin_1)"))
 (segment (start 111.39 89.85) (end 111.45 89.91) (width 0.2) (layer "B.Cu") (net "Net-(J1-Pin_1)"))
 (segment (start 180.8575 107.1) (end 183.205 107.1) (width 0.2) (layer "F.Cu") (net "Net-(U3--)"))
 (segment (start 183.8575 103.4475) (end 183.955 103.4475) (width 0.2) (layer "F.Cu") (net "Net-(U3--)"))
 (segment (start 183.205 107.1) (end 183.8575 106.4475) (width 0.2) (layer "F.Cu") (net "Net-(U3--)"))
 (segment (start 184.8575 105.4475) (end 183.8575 106.4475) (width 0.2) (layer "F.Cu") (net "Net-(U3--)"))
 (segment (start 183.955 103.4475) (end 184.8575 104.35) (width 0.2) (layer "F.Cu") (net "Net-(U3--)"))
 (segment (start 184.8575 104.35) (end 184.8575 105.4475) (width 0.2) (layer "F.Cu") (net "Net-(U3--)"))
 (segment (start 169.76 106.4475) (end 168.8575 107.35) (width 0.2) (layer "F.Cu") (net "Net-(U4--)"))
 (segment (start 172.3575 103.85) (end 169.76 106.4475) (width 0.2) (layer "F.Cu") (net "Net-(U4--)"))
 (segment (start 172.3575 106.4475) (end 169.76 106.4475) (width 0.2) (layer "F.Cu") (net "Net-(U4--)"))
 (segment (start 172.3575 102.35) (end 172.3575 103.85) (width 0.2) (layer "F.Cu") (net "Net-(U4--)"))
 (segment (start 104.5075 95.5) (end 104.3575 95.35) (width 0.2) (layer "B.Cu") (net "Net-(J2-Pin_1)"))
 (segment (start 111.45 95.5) (end 104.5075 95.5) (width 0.2) (layer "B.Cu") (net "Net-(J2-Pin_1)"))
 (segment (start 166.8575 106.85) (end 168.8575 104.85) (width 0.2) (layer "B.Cu") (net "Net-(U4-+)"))
 (segment (start 166.8575 110.35) (end 166.8575 106.85) (width 0.2) (layer "B.Cu") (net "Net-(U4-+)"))
 (segment (start 175.3575 112.35) (end 168.8575 112.35) (width 0.2) (layer "B.Cu") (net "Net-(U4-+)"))
 (segment (start 168.8575 112.35) (end 166.8575 110.35) (width 0.2) (layer "B.Cu") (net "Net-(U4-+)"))
 (segment (start 177.3575 110.35) (end 175.3575 112.35) (width 0.2) (layer "B.Cu") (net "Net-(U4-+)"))
 (segment (start 177.3575 108.35) (end 177.3575 110.35) (width 0.2) (layer "B.Cu") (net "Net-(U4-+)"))
 (segment (start 176.1075 107.1) (end 177.3575 108.35) (width 0.2) (layer "B.Cu") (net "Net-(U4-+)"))
 (segment (start 175.8575 107.1) (end 176.1075 107.1) (width 0.2) (layer "B.Cu") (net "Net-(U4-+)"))
 (segment (start 160.955 107.35) (end 163.8575 107.35) (width 0.2) (layer "F.Cu") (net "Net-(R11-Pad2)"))
 (segment (start 163.76 107.2525) (end 163.8575 107.35) (width 0.2) (layer "F.Cu") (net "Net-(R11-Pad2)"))
 (segment (start 159.735 107.325) (end 159.76 107.35) (width 0.2) (layer "F.Cu") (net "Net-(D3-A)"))
 (segment (start 157.8575 107.325) (end 159.735 107.325) (width 0.2) (layer "F.Cu") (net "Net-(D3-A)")))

